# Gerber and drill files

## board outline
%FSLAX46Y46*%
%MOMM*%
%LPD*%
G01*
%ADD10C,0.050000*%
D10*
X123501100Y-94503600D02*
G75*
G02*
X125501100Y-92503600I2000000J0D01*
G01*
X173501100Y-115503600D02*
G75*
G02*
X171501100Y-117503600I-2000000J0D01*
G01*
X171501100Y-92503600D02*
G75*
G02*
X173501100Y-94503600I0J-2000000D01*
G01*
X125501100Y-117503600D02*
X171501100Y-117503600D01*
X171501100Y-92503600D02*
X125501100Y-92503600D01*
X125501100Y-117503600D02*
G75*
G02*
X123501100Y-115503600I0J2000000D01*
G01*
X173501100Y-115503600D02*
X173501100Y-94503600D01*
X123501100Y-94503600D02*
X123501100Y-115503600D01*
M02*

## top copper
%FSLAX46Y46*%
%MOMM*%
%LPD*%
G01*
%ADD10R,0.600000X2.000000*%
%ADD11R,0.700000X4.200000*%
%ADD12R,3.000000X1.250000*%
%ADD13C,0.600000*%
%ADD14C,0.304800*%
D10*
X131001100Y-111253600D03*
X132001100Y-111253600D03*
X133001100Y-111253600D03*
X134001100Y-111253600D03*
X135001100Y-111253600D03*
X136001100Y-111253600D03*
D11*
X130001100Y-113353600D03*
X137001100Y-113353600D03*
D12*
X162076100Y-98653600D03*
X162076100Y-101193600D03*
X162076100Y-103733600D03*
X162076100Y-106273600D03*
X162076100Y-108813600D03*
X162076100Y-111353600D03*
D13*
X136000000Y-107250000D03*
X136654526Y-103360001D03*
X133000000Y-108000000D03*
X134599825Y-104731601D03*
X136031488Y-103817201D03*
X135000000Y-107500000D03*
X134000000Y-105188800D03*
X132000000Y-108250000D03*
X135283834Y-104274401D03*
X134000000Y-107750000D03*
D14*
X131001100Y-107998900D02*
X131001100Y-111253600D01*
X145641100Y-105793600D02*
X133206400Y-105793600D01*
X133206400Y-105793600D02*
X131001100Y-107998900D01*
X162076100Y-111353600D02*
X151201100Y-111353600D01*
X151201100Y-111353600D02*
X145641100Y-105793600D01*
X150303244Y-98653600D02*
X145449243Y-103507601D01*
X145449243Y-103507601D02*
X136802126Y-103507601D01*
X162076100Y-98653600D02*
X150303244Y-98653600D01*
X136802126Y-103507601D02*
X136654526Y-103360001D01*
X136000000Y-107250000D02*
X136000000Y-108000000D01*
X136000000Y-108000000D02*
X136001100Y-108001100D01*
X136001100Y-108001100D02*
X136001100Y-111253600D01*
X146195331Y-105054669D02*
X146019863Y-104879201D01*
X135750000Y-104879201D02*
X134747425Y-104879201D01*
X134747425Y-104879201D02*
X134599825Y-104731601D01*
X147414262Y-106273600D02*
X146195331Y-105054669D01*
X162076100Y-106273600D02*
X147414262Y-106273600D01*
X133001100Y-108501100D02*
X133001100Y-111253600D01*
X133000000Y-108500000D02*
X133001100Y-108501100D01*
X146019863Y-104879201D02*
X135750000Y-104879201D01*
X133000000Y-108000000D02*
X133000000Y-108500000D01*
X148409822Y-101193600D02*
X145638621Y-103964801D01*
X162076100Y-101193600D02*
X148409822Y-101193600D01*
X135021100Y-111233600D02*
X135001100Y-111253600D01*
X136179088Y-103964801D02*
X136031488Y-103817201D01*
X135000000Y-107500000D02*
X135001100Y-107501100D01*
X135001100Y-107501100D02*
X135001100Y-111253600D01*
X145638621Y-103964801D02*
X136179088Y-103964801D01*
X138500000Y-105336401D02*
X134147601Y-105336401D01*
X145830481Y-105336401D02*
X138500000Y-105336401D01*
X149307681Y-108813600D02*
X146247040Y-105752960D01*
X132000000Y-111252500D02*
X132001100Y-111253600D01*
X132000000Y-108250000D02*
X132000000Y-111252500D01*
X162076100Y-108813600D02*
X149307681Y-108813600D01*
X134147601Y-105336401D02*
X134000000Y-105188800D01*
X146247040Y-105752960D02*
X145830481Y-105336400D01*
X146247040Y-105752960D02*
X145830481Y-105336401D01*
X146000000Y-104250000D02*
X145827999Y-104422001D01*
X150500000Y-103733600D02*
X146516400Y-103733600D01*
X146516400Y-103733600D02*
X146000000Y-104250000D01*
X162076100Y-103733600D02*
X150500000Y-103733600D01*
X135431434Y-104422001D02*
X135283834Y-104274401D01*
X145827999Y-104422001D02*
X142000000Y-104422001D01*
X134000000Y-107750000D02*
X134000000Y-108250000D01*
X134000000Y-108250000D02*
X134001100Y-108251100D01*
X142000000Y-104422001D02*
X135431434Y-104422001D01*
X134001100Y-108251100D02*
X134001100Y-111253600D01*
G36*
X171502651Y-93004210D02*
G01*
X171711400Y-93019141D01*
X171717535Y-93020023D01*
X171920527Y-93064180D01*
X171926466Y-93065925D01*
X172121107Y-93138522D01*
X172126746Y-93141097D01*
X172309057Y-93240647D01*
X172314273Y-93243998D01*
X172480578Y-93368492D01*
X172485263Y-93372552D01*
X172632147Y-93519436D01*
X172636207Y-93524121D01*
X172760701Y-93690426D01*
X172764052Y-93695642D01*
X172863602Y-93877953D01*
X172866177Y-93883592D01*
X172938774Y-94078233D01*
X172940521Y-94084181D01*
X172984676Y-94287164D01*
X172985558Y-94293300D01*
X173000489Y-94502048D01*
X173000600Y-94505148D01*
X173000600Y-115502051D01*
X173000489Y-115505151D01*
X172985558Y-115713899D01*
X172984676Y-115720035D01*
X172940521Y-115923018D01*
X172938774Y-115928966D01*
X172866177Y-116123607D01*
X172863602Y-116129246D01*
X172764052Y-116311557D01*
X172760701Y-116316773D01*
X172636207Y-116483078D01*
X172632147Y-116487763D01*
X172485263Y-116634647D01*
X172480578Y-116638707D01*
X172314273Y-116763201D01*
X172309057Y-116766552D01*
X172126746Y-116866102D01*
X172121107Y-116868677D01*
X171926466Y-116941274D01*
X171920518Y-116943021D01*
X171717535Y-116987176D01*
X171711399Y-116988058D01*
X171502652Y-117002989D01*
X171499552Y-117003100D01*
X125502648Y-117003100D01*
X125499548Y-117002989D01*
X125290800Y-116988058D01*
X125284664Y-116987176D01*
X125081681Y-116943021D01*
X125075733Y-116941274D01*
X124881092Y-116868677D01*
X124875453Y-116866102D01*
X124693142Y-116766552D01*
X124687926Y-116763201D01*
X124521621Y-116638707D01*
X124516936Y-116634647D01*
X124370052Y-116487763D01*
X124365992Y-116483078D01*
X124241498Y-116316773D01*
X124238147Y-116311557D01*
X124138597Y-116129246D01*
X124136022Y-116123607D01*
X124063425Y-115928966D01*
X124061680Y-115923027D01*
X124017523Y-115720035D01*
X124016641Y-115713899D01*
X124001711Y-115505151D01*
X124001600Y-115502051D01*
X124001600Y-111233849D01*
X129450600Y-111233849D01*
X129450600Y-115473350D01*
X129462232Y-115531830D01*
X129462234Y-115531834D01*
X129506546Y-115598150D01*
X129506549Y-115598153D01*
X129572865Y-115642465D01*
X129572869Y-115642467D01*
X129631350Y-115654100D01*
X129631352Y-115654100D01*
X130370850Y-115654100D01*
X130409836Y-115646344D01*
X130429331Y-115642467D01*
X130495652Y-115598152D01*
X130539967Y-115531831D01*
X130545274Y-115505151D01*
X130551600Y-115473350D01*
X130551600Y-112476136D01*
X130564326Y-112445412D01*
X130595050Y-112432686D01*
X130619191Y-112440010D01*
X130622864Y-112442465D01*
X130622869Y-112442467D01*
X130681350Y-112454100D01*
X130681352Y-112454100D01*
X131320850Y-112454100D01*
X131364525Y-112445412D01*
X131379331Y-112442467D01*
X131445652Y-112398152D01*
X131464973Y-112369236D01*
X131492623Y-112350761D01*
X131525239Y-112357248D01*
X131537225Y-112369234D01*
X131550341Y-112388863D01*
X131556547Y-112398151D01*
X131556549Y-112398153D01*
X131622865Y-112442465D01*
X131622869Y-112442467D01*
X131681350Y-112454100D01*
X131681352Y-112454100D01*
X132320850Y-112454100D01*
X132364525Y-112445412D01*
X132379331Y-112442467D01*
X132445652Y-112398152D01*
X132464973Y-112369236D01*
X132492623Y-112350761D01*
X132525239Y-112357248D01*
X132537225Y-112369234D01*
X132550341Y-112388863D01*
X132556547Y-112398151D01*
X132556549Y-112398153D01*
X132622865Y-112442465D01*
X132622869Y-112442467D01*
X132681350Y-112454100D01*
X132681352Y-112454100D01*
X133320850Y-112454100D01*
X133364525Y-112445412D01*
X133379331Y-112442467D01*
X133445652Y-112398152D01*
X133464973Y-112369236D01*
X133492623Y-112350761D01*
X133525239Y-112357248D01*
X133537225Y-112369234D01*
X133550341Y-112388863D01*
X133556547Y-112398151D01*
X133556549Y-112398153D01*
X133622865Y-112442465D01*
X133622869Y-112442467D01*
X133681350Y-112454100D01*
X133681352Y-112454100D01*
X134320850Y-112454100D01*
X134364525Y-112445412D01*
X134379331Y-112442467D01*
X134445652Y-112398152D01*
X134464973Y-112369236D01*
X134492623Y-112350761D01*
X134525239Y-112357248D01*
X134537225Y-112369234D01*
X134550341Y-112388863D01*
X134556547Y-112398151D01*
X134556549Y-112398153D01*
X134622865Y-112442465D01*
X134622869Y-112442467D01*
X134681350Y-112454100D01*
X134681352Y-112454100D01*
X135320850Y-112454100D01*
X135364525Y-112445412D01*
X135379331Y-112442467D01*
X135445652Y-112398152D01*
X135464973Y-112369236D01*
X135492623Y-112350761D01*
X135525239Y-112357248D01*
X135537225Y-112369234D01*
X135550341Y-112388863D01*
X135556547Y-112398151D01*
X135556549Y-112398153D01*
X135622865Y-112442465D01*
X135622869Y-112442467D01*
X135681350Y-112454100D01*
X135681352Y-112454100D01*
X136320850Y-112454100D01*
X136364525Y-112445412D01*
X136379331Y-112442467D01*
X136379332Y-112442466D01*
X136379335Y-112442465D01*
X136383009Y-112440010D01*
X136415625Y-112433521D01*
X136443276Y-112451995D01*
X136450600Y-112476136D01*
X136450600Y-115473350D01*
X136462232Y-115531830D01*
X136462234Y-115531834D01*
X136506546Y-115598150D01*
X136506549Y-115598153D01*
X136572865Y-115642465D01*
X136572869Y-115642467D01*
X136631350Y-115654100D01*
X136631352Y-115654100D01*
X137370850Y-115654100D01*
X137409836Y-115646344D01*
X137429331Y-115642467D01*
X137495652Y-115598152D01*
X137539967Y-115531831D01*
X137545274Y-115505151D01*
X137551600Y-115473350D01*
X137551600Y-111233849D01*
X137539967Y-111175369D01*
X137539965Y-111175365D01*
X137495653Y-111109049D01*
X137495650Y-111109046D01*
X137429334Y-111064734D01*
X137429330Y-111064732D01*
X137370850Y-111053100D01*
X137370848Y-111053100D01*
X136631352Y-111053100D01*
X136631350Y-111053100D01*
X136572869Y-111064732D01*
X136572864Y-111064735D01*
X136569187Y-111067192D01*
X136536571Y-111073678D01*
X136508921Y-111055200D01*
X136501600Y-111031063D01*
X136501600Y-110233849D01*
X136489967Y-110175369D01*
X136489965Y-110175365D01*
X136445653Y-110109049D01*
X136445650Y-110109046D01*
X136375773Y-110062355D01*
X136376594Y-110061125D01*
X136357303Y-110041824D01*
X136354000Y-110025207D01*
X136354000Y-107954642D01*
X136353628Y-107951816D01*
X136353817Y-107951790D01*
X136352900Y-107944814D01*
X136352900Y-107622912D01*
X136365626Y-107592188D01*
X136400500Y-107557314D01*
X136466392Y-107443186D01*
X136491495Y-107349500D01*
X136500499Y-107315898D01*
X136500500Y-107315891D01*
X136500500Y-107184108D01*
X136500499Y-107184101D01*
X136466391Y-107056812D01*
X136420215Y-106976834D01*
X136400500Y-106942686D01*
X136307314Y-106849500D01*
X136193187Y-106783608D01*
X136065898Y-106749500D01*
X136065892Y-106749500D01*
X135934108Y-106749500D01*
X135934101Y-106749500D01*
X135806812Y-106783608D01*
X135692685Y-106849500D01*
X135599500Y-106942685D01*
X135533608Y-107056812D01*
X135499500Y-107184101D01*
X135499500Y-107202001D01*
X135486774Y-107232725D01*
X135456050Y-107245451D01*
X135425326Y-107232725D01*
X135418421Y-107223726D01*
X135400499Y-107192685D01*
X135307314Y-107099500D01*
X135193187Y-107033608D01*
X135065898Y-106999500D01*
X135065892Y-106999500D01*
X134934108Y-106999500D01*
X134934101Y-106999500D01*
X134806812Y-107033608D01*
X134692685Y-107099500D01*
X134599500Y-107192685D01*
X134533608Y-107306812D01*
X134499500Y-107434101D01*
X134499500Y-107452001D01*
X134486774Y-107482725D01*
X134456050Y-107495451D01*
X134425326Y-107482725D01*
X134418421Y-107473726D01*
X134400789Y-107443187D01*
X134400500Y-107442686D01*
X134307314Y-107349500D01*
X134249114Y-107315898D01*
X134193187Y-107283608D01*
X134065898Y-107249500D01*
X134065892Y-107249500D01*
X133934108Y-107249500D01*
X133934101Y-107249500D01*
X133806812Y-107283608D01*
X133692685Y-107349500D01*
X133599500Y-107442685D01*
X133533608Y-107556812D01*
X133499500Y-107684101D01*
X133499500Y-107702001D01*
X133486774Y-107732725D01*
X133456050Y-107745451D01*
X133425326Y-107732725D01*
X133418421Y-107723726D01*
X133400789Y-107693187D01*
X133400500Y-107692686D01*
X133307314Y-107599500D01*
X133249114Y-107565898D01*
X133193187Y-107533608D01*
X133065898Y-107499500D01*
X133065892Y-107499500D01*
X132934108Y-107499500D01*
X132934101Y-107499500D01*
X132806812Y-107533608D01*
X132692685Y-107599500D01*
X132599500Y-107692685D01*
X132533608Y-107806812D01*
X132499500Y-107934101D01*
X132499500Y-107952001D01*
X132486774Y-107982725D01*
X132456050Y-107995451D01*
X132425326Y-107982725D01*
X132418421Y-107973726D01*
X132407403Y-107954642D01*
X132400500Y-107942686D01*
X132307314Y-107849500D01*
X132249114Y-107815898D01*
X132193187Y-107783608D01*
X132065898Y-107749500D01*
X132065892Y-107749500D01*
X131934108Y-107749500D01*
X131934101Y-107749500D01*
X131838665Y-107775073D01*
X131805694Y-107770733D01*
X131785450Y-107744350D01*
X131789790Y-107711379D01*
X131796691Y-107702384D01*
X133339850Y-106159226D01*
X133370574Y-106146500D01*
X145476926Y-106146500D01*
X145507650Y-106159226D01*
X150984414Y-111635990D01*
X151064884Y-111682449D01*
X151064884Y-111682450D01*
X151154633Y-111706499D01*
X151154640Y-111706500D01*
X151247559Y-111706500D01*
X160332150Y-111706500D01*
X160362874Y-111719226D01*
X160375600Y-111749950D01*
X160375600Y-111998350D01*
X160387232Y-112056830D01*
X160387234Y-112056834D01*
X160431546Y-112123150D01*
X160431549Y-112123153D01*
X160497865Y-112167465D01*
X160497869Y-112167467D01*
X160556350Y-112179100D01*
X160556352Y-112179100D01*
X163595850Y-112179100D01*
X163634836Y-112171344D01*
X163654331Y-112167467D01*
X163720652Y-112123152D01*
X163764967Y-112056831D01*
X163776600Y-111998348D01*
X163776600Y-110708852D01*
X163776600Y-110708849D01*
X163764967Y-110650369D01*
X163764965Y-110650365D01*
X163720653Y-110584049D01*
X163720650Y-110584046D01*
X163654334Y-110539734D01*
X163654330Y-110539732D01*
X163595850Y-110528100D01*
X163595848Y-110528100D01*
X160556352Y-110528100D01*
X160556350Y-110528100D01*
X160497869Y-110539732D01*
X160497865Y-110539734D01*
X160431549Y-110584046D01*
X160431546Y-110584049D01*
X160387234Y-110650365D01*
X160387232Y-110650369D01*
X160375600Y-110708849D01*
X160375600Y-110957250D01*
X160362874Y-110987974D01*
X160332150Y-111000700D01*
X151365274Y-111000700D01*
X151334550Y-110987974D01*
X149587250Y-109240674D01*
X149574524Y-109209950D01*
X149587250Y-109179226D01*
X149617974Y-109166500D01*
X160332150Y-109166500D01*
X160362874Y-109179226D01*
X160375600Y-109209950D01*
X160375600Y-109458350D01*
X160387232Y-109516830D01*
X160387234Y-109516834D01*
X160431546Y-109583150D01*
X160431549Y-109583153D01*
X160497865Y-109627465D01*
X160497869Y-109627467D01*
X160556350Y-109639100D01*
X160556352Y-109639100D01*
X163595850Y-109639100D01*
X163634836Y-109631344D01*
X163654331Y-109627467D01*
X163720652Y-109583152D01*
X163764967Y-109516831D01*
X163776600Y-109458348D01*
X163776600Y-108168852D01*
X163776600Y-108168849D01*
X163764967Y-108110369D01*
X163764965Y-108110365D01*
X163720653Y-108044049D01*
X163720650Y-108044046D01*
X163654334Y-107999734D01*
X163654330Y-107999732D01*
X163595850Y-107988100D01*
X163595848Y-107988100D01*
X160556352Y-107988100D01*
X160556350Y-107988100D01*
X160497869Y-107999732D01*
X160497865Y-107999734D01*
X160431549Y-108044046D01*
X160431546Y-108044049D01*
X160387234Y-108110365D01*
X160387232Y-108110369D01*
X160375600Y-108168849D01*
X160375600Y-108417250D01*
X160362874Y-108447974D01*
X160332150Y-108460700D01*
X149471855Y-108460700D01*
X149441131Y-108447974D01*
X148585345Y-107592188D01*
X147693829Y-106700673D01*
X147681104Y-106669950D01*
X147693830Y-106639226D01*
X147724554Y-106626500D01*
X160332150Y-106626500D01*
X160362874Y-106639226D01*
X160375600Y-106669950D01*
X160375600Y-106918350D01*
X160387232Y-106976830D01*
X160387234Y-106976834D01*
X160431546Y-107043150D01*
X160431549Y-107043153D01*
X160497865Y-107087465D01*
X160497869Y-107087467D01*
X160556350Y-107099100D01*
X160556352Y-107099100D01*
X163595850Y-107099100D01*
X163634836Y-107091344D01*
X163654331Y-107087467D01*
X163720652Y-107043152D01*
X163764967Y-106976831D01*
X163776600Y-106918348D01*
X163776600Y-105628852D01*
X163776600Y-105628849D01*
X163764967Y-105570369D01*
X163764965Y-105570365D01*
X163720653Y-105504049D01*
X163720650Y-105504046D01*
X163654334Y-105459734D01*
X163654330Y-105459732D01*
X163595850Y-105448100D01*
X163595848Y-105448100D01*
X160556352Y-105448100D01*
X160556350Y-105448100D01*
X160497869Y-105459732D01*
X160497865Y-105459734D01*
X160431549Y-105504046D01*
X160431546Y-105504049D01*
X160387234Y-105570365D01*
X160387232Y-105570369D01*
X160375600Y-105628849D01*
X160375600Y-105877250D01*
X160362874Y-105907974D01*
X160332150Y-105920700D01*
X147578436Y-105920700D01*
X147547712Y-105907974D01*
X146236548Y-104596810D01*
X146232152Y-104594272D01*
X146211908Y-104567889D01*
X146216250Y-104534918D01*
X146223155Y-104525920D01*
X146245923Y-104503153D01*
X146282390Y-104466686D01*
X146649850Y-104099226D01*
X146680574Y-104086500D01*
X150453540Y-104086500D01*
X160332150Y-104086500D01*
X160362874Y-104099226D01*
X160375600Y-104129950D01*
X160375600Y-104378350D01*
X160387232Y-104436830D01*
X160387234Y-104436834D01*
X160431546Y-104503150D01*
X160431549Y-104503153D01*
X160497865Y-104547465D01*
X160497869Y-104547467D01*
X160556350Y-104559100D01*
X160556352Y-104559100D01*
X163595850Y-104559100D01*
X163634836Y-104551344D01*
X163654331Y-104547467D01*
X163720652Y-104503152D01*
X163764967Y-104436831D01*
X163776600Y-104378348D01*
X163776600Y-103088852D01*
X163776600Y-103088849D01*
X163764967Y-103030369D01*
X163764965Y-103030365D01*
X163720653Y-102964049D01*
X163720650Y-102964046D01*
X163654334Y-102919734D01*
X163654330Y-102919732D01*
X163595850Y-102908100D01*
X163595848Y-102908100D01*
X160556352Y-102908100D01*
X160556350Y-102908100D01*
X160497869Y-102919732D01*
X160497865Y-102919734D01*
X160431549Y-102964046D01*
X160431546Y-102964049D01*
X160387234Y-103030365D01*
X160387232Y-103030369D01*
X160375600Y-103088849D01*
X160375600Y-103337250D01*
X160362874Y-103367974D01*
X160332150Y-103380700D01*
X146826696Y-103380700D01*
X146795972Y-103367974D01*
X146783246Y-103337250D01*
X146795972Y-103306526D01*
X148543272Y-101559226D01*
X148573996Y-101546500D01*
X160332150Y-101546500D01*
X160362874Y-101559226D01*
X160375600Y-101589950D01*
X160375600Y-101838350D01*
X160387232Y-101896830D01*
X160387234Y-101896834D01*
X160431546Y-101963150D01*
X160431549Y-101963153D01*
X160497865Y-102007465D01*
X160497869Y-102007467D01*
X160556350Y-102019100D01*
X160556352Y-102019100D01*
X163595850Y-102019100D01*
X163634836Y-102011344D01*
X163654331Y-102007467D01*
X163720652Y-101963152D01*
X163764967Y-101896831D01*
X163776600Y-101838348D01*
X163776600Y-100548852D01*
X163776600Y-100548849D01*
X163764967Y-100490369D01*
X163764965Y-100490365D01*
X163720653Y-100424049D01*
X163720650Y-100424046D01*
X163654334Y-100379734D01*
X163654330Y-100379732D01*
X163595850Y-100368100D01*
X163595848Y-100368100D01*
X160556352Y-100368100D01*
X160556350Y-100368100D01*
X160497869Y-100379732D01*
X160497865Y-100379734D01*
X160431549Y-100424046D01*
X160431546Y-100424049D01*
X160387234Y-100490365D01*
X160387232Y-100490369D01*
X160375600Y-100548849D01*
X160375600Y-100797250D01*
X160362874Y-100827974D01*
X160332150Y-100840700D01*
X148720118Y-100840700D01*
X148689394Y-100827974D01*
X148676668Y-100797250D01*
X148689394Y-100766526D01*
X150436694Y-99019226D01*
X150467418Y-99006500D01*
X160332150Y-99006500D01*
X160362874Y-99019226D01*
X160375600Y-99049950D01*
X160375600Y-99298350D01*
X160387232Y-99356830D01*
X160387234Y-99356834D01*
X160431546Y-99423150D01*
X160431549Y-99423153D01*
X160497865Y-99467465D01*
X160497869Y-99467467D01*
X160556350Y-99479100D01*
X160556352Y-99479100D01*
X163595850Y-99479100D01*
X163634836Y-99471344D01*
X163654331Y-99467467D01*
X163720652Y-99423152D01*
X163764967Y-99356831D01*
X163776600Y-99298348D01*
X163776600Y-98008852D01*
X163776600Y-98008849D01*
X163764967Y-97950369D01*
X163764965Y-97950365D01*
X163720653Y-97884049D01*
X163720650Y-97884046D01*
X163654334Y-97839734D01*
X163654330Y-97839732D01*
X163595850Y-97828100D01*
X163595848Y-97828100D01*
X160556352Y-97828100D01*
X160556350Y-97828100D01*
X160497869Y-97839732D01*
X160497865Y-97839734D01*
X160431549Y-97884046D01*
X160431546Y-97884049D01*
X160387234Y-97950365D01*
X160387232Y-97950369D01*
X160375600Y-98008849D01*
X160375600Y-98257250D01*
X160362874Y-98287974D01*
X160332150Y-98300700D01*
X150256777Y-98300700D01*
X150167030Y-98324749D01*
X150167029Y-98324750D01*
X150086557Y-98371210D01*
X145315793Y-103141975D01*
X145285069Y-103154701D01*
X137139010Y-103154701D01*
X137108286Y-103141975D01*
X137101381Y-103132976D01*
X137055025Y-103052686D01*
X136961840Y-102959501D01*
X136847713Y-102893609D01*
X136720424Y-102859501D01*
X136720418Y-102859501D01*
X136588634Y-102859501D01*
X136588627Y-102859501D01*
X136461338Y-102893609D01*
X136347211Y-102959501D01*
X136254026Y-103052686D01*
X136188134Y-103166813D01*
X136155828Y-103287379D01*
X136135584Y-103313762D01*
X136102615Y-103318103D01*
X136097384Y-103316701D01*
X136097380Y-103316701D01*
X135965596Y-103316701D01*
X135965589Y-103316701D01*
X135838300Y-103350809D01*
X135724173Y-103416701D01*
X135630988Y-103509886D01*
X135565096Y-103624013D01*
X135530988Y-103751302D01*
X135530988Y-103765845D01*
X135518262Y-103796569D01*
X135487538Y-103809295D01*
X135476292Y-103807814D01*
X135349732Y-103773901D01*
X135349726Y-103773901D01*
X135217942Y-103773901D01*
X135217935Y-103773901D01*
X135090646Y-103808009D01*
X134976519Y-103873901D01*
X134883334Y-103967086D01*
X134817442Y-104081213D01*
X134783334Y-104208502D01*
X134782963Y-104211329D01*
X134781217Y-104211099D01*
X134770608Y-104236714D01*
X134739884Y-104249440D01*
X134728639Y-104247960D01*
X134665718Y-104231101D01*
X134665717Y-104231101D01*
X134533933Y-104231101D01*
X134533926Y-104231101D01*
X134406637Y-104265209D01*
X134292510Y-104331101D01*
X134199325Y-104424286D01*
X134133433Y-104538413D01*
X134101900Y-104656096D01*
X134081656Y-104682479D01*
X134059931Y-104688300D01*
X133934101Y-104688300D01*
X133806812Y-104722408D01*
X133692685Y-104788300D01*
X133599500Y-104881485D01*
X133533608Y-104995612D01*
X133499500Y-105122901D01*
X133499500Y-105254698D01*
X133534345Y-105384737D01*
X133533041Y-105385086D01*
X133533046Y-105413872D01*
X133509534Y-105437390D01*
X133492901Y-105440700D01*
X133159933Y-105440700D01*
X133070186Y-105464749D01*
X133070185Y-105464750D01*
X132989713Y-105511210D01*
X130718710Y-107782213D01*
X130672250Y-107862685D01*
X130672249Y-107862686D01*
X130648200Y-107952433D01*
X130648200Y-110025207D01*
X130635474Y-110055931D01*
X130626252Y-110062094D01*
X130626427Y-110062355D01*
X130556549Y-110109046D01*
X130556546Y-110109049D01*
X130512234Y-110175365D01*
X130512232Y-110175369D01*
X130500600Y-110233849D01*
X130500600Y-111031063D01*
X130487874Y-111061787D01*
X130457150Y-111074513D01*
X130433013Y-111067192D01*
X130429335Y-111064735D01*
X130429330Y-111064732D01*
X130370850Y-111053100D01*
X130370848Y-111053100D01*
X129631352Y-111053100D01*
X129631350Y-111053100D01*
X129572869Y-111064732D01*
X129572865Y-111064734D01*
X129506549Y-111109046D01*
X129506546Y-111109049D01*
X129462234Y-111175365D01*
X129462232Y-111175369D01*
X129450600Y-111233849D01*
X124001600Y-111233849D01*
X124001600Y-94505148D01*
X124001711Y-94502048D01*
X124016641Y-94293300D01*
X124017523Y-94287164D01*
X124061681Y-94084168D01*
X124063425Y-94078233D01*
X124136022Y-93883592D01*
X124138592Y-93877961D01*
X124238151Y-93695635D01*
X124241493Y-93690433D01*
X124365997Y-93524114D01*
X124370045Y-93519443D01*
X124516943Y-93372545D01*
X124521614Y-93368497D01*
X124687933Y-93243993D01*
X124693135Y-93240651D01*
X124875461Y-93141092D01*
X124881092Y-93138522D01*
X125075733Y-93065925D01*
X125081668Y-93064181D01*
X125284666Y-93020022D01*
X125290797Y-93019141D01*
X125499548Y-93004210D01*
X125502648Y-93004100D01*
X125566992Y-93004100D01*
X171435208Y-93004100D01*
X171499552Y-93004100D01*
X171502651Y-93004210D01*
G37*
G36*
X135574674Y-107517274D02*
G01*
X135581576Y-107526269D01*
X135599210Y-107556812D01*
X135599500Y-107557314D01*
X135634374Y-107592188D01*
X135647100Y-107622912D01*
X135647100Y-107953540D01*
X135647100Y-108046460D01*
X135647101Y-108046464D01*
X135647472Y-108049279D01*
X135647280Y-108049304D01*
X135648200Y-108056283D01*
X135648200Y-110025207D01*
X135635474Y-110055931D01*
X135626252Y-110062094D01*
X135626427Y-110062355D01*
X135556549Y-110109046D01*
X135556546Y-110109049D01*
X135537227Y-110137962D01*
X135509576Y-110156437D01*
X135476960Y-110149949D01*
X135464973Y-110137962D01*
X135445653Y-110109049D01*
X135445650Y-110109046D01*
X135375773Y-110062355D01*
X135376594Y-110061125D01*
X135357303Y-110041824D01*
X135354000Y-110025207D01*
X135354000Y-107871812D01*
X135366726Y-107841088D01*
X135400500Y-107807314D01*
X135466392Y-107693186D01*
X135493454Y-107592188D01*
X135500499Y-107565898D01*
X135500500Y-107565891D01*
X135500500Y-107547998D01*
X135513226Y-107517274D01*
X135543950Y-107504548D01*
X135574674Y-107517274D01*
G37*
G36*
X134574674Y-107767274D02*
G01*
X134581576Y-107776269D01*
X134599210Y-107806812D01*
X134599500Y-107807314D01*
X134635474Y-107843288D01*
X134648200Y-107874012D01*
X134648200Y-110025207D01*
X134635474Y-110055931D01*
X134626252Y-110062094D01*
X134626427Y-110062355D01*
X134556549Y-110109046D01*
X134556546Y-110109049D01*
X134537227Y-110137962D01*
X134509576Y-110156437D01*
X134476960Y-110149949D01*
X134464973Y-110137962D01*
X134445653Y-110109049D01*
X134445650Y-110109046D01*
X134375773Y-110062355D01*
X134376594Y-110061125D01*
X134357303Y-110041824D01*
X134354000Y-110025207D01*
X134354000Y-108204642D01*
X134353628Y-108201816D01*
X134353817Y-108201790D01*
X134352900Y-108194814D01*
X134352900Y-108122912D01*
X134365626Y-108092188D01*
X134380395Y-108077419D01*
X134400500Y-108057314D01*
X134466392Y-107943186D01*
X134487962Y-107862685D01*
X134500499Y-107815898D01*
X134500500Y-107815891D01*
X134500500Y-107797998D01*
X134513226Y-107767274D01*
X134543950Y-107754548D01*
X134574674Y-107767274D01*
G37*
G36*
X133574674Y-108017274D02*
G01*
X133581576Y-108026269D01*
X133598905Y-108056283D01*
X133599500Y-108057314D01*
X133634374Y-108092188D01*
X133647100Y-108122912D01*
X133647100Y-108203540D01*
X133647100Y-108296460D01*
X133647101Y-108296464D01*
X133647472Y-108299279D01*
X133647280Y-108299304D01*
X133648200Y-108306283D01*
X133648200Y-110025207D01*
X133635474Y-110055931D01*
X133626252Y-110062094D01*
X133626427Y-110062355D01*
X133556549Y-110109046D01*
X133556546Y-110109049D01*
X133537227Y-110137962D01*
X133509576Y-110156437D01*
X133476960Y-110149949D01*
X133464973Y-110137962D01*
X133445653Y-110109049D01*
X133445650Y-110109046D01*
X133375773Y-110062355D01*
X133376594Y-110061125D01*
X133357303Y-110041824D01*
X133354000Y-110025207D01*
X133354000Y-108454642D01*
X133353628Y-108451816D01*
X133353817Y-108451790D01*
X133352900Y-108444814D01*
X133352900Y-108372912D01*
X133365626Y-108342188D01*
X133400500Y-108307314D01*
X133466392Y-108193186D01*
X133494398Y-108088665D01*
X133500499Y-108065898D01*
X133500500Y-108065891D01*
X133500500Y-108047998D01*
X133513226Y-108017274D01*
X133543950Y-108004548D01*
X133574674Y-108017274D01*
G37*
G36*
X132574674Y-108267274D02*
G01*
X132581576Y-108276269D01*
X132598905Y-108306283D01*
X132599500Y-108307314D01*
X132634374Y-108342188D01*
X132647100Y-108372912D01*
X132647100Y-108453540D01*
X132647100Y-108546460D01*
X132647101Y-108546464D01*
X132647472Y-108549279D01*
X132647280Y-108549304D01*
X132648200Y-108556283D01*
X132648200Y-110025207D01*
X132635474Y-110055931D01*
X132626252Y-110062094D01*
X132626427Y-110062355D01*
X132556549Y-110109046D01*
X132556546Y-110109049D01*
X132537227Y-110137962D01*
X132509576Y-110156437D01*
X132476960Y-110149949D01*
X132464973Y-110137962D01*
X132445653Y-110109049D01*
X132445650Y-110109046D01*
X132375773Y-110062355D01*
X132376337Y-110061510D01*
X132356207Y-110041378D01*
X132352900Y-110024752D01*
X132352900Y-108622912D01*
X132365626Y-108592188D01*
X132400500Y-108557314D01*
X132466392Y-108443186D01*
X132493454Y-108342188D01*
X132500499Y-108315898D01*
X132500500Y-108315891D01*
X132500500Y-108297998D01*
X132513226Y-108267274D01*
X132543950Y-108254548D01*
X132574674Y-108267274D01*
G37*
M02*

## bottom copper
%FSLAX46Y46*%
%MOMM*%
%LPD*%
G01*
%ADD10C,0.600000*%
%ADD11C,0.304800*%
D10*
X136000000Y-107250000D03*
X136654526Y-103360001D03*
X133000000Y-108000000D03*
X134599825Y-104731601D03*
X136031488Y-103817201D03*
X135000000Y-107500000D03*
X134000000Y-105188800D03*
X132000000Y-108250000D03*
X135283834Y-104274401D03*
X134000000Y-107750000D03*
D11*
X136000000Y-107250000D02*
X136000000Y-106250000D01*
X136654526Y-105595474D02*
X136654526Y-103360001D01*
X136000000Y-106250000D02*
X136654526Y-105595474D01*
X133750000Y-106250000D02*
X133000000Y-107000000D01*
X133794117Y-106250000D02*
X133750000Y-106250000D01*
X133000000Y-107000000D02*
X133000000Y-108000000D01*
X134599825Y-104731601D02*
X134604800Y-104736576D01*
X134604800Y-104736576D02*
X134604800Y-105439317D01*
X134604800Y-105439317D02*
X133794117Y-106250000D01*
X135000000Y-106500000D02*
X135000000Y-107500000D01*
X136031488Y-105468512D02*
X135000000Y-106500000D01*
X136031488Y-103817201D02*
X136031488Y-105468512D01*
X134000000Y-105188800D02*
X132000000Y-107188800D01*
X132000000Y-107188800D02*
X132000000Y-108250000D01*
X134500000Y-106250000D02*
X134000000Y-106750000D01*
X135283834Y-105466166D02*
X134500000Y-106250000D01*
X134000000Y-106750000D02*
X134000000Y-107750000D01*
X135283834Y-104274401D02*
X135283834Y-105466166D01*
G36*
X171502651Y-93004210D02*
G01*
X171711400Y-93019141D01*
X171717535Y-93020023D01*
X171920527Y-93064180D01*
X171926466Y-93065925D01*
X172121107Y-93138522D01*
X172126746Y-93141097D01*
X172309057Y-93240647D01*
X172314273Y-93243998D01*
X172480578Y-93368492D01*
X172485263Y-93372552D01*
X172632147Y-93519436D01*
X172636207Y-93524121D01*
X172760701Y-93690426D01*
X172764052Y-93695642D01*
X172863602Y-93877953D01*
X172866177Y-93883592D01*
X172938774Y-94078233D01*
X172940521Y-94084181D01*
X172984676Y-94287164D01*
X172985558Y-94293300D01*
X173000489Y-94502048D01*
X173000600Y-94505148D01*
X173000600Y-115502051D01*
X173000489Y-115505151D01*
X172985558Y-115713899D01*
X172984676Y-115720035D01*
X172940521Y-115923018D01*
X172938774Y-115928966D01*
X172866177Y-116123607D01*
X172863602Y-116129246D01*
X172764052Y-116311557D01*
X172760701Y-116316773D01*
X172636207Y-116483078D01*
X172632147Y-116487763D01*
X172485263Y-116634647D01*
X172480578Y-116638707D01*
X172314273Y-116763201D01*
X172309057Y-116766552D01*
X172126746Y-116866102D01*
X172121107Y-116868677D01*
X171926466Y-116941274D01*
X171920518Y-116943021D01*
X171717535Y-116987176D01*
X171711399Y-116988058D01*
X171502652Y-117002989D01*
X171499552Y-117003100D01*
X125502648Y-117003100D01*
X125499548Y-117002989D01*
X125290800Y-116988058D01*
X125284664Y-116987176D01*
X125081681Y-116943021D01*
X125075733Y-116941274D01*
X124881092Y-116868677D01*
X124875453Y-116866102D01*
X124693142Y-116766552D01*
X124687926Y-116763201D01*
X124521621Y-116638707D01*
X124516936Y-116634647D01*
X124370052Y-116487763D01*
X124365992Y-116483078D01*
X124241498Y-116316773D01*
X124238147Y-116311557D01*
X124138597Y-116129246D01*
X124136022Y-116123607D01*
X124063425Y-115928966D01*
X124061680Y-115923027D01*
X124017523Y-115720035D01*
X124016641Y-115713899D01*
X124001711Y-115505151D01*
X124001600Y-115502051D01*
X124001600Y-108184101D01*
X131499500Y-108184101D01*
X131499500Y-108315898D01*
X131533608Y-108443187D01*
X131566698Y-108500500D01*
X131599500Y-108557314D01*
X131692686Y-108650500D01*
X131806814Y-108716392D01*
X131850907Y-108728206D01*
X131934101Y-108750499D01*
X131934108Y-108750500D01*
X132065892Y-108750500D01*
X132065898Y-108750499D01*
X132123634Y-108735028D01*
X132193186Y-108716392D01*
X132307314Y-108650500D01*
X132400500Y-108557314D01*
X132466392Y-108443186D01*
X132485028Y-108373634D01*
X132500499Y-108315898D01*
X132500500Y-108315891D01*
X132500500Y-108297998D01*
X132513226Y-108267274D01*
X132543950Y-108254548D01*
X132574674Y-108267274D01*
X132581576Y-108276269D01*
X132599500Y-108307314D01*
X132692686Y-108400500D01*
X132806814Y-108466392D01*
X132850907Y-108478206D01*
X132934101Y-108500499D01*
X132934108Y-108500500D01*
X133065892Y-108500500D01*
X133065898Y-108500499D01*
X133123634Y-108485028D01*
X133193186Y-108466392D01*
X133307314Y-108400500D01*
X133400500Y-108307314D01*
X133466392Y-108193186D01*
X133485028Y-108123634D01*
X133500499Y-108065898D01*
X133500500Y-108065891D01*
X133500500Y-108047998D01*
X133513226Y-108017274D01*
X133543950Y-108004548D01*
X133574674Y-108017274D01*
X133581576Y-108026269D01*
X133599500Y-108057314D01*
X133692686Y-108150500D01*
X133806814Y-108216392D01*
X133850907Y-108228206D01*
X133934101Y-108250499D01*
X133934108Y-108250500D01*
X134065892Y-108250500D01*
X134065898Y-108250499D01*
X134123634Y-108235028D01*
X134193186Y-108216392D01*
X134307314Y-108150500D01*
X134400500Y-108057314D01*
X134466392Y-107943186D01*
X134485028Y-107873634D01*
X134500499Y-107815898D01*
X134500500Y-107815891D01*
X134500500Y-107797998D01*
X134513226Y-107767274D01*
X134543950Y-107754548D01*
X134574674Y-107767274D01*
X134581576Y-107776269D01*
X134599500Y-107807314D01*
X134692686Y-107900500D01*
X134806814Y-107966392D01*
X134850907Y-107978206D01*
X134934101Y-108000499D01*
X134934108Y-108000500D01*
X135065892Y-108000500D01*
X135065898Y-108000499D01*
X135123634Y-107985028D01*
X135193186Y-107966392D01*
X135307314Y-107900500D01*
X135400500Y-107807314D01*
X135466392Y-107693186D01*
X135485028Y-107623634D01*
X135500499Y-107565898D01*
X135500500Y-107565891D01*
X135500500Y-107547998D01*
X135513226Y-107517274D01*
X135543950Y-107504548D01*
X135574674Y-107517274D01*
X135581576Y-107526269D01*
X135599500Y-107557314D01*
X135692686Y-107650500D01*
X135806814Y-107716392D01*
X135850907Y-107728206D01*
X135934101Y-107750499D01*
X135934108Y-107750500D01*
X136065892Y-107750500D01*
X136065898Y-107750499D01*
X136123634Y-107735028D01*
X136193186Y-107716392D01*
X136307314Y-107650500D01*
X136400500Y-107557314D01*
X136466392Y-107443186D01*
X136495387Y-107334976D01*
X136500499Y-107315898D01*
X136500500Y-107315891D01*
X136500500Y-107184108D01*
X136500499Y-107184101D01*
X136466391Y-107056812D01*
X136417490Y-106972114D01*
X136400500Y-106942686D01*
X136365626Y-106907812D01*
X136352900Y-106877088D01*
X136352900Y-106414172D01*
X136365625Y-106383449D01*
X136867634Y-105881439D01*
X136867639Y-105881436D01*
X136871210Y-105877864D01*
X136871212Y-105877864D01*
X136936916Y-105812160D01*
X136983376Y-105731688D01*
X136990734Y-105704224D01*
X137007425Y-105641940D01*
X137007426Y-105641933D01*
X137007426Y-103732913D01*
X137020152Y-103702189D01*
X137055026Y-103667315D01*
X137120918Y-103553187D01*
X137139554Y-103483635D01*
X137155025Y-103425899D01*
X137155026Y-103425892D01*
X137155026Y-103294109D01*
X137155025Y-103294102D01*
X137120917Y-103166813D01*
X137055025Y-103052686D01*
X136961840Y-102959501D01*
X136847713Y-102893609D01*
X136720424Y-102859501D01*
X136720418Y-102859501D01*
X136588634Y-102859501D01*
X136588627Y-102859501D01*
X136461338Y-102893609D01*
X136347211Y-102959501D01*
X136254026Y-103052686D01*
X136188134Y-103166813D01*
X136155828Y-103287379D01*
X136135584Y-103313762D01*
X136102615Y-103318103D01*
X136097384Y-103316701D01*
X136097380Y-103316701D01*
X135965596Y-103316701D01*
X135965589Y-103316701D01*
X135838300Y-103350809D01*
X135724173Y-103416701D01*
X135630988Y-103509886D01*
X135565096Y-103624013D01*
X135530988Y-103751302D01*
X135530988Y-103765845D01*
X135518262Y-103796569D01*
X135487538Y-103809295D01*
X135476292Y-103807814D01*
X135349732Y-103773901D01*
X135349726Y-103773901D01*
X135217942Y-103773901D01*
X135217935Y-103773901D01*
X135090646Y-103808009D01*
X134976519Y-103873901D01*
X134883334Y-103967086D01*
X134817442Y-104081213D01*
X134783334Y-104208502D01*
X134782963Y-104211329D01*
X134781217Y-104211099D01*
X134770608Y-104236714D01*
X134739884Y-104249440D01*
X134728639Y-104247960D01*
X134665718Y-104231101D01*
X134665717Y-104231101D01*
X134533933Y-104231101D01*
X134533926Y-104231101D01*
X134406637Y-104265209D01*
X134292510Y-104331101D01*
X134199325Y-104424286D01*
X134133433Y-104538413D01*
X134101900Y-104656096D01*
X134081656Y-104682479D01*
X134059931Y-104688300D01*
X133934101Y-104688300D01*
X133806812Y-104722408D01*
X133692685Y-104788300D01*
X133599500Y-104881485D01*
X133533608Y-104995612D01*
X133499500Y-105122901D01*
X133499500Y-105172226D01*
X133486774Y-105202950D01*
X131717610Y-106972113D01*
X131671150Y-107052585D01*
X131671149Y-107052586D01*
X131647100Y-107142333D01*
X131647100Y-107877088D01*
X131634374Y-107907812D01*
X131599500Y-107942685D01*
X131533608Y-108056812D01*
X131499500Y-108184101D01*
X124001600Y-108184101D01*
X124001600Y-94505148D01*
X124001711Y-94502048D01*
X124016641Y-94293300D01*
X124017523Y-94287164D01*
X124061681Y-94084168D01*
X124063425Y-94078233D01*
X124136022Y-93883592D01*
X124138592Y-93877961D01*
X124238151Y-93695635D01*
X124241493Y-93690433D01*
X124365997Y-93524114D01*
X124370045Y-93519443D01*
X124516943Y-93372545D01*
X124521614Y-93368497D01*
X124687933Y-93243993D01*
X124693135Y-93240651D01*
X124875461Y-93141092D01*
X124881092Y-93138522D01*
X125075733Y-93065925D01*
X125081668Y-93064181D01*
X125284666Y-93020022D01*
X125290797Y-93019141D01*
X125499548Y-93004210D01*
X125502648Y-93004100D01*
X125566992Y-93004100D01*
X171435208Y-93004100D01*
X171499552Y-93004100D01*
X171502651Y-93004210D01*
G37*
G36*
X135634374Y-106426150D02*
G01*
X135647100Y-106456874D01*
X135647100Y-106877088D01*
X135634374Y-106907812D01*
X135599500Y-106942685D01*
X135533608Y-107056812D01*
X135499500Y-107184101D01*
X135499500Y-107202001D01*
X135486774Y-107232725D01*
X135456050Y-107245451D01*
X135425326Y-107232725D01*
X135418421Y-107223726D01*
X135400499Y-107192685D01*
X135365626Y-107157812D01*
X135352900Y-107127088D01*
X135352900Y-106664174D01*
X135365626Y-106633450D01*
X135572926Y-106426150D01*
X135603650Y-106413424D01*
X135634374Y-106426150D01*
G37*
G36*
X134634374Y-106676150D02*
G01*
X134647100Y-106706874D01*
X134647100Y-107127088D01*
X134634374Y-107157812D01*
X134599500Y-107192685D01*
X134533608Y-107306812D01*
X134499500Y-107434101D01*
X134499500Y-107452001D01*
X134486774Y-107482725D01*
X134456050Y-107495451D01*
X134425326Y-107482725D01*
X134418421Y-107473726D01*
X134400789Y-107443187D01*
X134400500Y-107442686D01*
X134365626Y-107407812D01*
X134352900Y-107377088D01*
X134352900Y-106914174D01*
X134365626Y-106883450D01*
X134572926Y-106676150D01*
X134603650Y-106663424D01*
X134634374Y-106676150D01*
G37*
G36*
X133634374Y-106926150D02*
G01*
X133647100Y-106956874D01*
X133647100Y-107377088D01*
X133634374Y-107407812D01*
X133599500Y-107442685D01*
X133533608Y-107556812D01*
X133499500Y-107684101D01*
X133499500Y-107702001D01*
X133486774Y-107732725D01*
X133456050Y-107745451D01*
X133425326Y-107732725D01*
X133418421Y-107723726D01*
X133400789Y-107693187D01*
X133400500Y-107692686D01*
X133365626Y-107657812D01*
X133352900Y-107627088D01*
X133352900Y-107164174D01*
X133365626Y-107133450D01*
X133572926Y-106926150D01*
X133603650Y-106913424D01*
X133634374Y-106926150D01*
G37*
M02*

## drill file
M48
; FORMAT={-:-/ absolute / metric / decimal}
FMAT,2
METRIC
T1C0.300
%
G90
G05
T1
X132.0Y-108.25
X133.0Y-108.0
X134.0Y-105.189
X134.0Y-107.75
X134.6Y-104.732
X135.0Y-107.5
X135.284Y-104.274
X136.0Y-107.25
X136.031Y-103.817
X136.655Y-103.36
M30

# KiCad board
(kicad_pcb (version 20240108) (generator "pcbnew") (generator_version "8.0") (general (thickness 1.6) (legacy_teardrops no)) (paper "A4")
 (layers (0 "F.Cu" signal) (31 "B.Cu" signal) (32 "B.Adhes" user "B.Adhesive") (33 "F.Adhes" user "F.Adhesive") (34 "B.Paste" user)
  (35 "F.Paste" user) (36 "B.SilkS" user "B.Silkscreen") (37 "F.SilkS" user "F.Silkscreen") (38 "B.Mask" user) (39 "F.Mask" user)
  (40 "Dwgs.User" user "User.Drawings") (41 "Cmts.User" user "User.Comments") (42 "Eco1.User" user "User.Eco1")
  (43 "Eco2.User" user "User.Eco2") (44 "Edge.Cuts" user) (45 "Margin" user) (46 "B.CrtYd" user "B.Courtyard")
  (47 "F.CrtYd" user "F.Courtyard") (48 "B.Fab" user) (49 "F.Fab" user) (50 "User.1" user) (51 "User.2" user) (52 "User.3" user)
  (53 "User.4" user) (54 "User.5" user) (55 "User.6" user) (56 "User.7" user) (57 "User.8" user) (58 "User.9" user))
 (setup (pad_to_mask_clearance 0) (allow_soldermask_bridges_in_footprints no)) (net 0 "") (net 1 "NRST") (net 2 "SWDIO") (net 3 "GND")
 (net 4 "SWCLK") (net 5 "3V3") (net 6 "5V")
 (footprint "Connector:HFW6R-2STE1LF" (layer "F.Cu") (at 133.5011 114.5036)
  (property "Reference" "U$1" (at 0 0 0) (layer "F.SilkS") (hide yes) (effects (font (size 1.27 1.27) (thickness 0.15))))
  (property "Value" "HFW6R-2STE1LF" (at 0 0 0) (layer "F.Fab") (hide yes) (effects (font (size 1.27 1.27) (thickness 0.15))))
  (pad "P$1" smd rect (at -2.5 -3.25) (size 0.6 2) (layers "F.Cu" "F.Paste" "F.Mask") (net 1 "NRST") (solder_mask_margin 0.0508)
   (thermal_bridge_angle 0))
  (pad "P$2" smd rect (at -1.5 -3.25) (size 0.6 2) (layers "F.Cu" "F.Paste" "F.Mask") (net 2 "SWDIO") (solder_mask_margin 0.0508)
   (thermal_bridge_angle 0))
  (pad "P$3" smd rect (at -0.5 -3.25) (size 0.6 2) (layers "F.Cu" "F.Paste" "F.Mask") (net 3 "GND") (solder_mask_margin 0.0508)
   (thermal_bridge_angle 0))
  (pad "P$4" smd rect (at 0.5 -3.25) (size 0.6 2) (layers "F.Cu" "F.Paste" "F.Mask") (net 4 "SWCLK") (solder_mask_margin 0.0508)
   (thermal_bridge_angle 0))
  (pad "P$5" smd rect (at 1.5 -3.25) (size 0.6 2) (layers "F.Cu" "F.Paste" "F.Mask") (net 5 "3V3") (solder_mask_margin 0.0508)
   (thermal_bridge_angle 0))
  (pad "P$6" smd rect (at 2.5 -3.25) (size 0.6 2) (layers "F.Cu" "F.Paste" "F.Mask") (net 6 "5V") (solder_mask_margin 0.0508)
   (thermal_bridge_angle 0))
  (pad "P$7" smd rect (at -3.5 -1.15) (size 0.7 4.2) (layers "F.Cu" "F.Paste" "F.Mask") (solder_mask_margin 0.0508) (thermal_bridge_angle 0))
  (pad "P$8" smd rect (at 3.5 -1.15) (size 0.7 4.2) (layers "F.Cu" "F.Paste" "F.Mask") (solder_mask_margin 0.0508) (thermal_bridge_angle 0)))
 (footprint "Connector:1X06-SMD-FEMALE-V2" (layer "F.Cu") (at 165.5011 105.0036 90)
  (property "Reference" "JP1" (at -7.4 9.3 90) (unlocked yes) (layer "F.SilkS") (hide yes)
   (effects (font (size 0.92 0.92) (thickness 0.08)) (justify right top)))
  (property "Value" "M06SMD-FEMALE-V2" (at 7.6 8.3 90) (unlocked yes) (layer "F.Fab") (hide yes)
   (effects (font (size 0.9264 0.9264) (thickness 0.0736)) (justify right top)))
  (pad "1" smd rect (at 6.35 -3.425 270) (size 1.25 3) (layers "F.Cu" "F.Paste" "F.Mask") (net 6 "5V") (solder_mask_margin 0.0508)
   (thermal_bridge_angle 0))
  (pad "2" smd rect (at 3.81 -3.425 270) (size 1.25 3) (layers "F.Cu" "F.Paste" "F.Mask") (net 5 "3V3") (solder_mask_margin 0.0508)
   (thermal_bridge_angle 0))
  (pad "3" smd rect (at 1.27 -3.425 270) (size 1.25 3) (layers "F.Cu" "F.Paste" "F.Mask") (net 4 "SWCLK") (solder_mask_margin 0.0508)
   (thermal_bridge_angle 0))
  (pad "4" smd rect (at -1.27 -3.425 270) (size 1.25 3) (layers "F.Cu" "F.Paste" "F.Mask") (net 3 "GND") (solder_mask_margin 0.0508)
   (thermal_bridge_angle 0))
  (pad "5" smd rect (at -3.81 -3.425 270) (size 1.25 3) (layers "F.Cu" "F.Paste" "F.Mask") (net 2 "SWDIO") (solder_mask_margin 0.0508)
   (thermal_bridge_angle 0))
  (pad "6" smd rect (at -6.35 -3.425 270) (size 1.25 3) (layers "F.Cu" "F.Paste" "F.Mask") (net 1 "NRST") (solder_mask_margin 0.0508)
   (thermal_bridge_angle 0)))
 (gr_arc (start 123.5011 94.5036) (mid 124.086886 93.089386) (end 125.5011 92.5036) (stroke (width 0.05) (type solid)) (layer "Edge.Cuts"))
 (gr_arc (start 173.5011 115.5036) (mid 172.915314 116.917814) (end 171.5011 117.5036) (stroke (width 0.05) (type solid))
  (layer "Edge.Cuts"))
 (gr_arc (start 171.5011 92.5036) (mid 172.915314 93.089386) (end 173.5011 94.5036) (stroke (width 0.05) (type solid)) (layer "Edge.Cuts"))
 (gr_line (start 125.5011 117.5036) (end 171.5011 117.5036) (stroke (width 0.05) (type solid)) (layer "Edge.Cuts"))
 (gr_line (start 171.5011 92.5036) (end 125.5011 92.5036) (stroke (width 0.05) (type solid)) (layer "Edge.Cuts"))
 (gr_arc (start 125.5011 117.5036) (mid 124.086886 116.917814) (end 123.5011 115.5036) (stroke (width 0.05) (type solid))
  (layer "Edge.Cuts"))
 (gr_line (start 173.5011 115.5036) (end 173.5011 94.5036) (stroke (width 0.05) (type solid)) (layer "Edge.Cuts"))
 (gr_line (start 123.5011 94.5036) (end 123.5011 115.5036) (stroke (width 0.05) (type solid)) (layer "Edge.Cuts"))
 (segment (start 131.0011 107.9989) (end 131.0011 111.2536) (width 0.3048) (layer "F.Cu") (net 1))
 (segment (start 145.6411 105.7936) (end 133.2064 105.7936) (width 0.3048) (layer "F.Cu") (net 1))
 (segment (start 133.2064 105.7936) (end 131.0011 107.9989) (width 0.3048) (layer "F.Cu") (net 1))
 (segment (start 162.0761 111.3536) (end 151.2011 111.3536) (width 0.3048) (layer "F.Cu") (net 1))
 (segment (start 151.2011 111.3536) (end 145.6411 105.7936) (width 0.3048) (layer "F.Cu") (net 1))
 (segment (start 150.303244 98.6536) (end 145.449243 103.507601) (width 0.3048) (layer "F.Cu") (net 6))
 (segment (start 145.449243 103.507601) (end 136.802126 103.507601) (width 0.3048) (layer "F.Cu") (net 6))
 (segment (start 162.0761 98.6536) (end 150.303244 98.6536) (width 0.3048) (layer "F.Cu") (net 6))
 (segment (start 136.802126 103.507601) (end 136.654526 103.360001) (width 0.3048) (layer "F.Cu") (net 6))
 (segment (start 136 107.25) (end 136 108) (width 0.3048) (layer "F.Cu") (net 6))
 (segment (start 136 108) (end 136.0011 108.0011) (width 0.3048) (layer "F.Cu") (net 6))
 (segment (start 136.0011 108.0011) (end 136.0011 111.2536) (width 0.3048) (layer "F.Cu") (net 6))
 (via (at 136 107.25) (size 0.6) (drill 0.3) (layers "F.Cu" "B.Cu") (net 6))
 (via (at 136.654526 103.360001) (size 0.6) (drill 0.3) (layers "F.Cu" "B.Cu") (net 6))
 (segment (start 136 107.25) (end 136 106.25) (width 0.3048) (layer "B.Cu") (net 6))
 (segment (start 136.654526 105.595474) (end 136.654526 103.360001) (width 0.3048) (layer "B.Cu") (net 6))
 (segment (start 136 106.25) (end 136.654526 105.595474) (width 0.3048) (layer "B.Cu") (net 6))
 (segment (start 146.195331 105.054669) (end 146.019863 104.879201) (width 0.3048) (layer "F.Cu") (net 3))
 (segment (start 135.75 104.879201) (end 134.747425 104.879201) (width 0.3048) (layer "F.Cu") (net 3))
 (segment (start 134.747425 104.879201) (end 134.599825 104.731601) (width 0.3048) (layer "F.Cu") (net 3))
 (segment (start 147.414262 106.2736) (end 146.195331 105.054669) (width 0.3048) (layer "F.Cu") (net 3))
 (segment (start 162.0761 106.2736) (end 147.414262 106.2736) (width 0.3048) (layer "F.Cu") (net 3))
 (segment (start 133.0011 108.5011) (end 133.0011 111.2536) (width 0.3048) (layer "F.Cu") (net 3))
 (segment (start 133 108.5) (end 133.0011 108.5011) (width 0.3048) (layer "F.Cu") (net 3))
 (segment (start 146.019863 104.879201) (end 135.75 104.879201) (width 0.3048) (layer "F.Cu") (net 3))
 (segment (start 133 108) (end 133 108.5) (width 0.3048) (layer "F.Cu") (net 3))
 (via (at 133 108) (size 0.6) (drill 0.3) (layers "F.Cu" "B.Cu") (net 3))
 (via (at 134.599825 104.731601) (size 0.6) (drill 0.3) (layers "F.Cu" "B.Cu") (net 3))
 (segment (start 133.75 106.25) (end 133 107) (width 0.3048) (layer "B.Cu") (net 3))
 (segment (start 133.794117 106.25) (end 133.75 106.25) (width 0.3048) (layer "B.Cu") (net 3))
 (segment (start 133 107) (end 133 108) (width 0.3048) (layer "B.Cu") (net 3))
 (segment (start 134.599825 104.731601) (end 134.6048 104.736576) (width 0.3048) (layer "B.Cu") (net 3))
 (segment (start 134.6048 104.736576) (end 134.6048 105.439317) (width 0.3048) (layer "B.Cu") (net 3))
 (segment (start 134.6048 105.439317) (end 133.794117 106.25) (width 0.3048) (layer "B.Cu") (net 3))
 (segment (start 148.409822 101.1936) (end 145.638621 103.964801) (width 0.3048) (layer "F.Cu") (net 5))
 (segment (start 162.0761 101.1936) (end 148.409822 101.1936) (width 0.3048) (layer "F.Cu") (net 5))
 (segment (start 135.0211 111.2336) (end 135.0011 111.2536) (width 0.3048) (layer "F.Cu") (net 5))
 (segment (start 136.179088 103.964801) (end 136.031488 103.817201) (width 0.3048) (layer "F.Cu") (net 5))
 (segment (start 135 107.5) (end 135.0011 107.5011) (width 0.3048) (layer "F.Cu") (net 5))
 (segment (start 135.0011 107.5011) (end 135.0011 111.2536) (width 0.3048) (layer "F.Cu") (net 5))
 (segment (start 145.638621 103.964801) (end 136.179088 103.964801) (width 0.3048) (layer "F.Cu") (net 5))
 (via (at 136.031488 103.817201) (size 0.6) (drill 0.3) (layers "F.Cu" "B.Cu") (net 5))
 (via (at 135 107.5) (size 0.6) (drill 0.3) (layers "F.Cu" "B.Cu") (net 5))
 (segment (start 135 106.5) (end 135 107.5) (width 0.3048) (layer "B.Cu") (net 5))
 (segment (start 136.031488 105.468512) (end 135 106.5) (width 0.3048) (layer "B.Cu") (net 5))
 (segment (start 136.031488 103.817201) (end 136.031488 105.468512) (width 0.3048) (layer "B.Cu") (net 5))
 (segment (start 138.5 105.336401) (end 134.147601 105.336401) (width 0.3048) (layer "F.Cu") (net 2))
 (segment (start 145.830481 105.336401) (end 138.5 105.336401) (width 0.3048) (layer "F.Cu") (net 2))
 (segment (start 149.307681 108.8136) (end 146.24704 105.75296) (width 0.3048) (layer "F.Cu") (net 2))
 (segment (start 132 111.2525) (end 132.0011 111.2536) (width 0.3048) (layer "F.Cu") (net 2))
 (segment (start 132 108.25) (end 132 111.2525) (width 0.3048) (layer "F.Cu") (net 2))
 (segment (start 162.0761 108.8136) (end 149.307681 108.8136) (width 0.3048) (layer "F.Cu") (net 2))
 (segment (start 134.147601 105.336401) (end 134 105.1888) (width 0.3048) (layer "F.Cu") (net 2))
 (segment (start 146.24704 105.75296) (end 145.830481 105.3364) (width 0.3048) (layer "F.Cu") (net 2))
 (segment (start 146.24704 105.75296) (end 145.830481 105.336401) (width 0.3048) (layer "F.Cu") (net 2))
 (via (at 134 105.1888) (size 0.6) (drill 0.3) (layers "F.Cu" "B.Cu") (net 2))
 (via (at 132 108.25) (size 0.6) (drill 0.3) (layers "F.Cu" "B.Cu") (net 2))
 (segment (start 134 105.1888) (end 132 107.1888) (width 0.3048) (layer "B.Cu") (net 2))
 (segment (start 132 107.1888) (end 132 108.25) (width 0.3048) (layer "B.Cu") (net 2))
 (segment (start 146 104.25) (end 145.827999 104.422001) (width 0.3048) (layer "F.Cu") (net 4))
 (segment (start 150.5 103.7336) (end 146.5164 103.7336) (width 0.3048) (layer "F.Cu") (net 4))
 (segment (start 146.5164 103.7336) (end 146 104.25) (width 0.3048) (layer "F.Cu") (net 4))
 (segment (start 162.0761 103.7336) (end 150.5 103.7336) (width 0.3048) (layer "F.Cu") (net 4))
 (segment (start 135.431434 104.422001) (end 135.283834 104.274401) (width 0.3048) (layer "F.Cu") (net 4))
 (segment (start 145.827999 104.422001) (end 142 104.422001) (width 0.3048) (layer "F.Cu") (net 4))
 (segment (start 134 107.75) (end 134 108.25) (width 0.3048) (layer "F.Cu") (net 4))
 (segment (start 134 108.25) (end 134.0011 108.2511) (width 0.3048) (layer "F.Cu") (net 4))
 (segment (start 142 104.422001) (end 135.431434 104.422001) (width 0.3048) (layer "F.Cu") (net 4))
 (segment (start 134.0011 108.2511) (end 134.0011 111.2536) (width 0.3048) (layer "F.Cu") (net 4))
 (via (at 135.283834 104.274401) (size 0.6) (drill 0.3) (layers "F.Cu" "B.Cu") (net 4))
 (via (at 134 107.75) (size 0.6) (drill 0.3) (layers "F.Cu" "B.Cu") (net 4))
 (segment (start 134.5 106.25) (end 134 106.75) (width 0.3048) (layer "B.Cu") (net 4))
 (segment (start 135.283834 105.466166) (end 134.5 106.25) (width 0.3048) (layer "B.Cu") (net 4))
 (segment (start 134 106.75) (end 134 107.75) (width 0.3048) (layer "B.Cu") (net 4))
 (segment (start 135.283834 104.274401) (end 135.283834 105.466166) (width 0.3048) (layer "B.Cu") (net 4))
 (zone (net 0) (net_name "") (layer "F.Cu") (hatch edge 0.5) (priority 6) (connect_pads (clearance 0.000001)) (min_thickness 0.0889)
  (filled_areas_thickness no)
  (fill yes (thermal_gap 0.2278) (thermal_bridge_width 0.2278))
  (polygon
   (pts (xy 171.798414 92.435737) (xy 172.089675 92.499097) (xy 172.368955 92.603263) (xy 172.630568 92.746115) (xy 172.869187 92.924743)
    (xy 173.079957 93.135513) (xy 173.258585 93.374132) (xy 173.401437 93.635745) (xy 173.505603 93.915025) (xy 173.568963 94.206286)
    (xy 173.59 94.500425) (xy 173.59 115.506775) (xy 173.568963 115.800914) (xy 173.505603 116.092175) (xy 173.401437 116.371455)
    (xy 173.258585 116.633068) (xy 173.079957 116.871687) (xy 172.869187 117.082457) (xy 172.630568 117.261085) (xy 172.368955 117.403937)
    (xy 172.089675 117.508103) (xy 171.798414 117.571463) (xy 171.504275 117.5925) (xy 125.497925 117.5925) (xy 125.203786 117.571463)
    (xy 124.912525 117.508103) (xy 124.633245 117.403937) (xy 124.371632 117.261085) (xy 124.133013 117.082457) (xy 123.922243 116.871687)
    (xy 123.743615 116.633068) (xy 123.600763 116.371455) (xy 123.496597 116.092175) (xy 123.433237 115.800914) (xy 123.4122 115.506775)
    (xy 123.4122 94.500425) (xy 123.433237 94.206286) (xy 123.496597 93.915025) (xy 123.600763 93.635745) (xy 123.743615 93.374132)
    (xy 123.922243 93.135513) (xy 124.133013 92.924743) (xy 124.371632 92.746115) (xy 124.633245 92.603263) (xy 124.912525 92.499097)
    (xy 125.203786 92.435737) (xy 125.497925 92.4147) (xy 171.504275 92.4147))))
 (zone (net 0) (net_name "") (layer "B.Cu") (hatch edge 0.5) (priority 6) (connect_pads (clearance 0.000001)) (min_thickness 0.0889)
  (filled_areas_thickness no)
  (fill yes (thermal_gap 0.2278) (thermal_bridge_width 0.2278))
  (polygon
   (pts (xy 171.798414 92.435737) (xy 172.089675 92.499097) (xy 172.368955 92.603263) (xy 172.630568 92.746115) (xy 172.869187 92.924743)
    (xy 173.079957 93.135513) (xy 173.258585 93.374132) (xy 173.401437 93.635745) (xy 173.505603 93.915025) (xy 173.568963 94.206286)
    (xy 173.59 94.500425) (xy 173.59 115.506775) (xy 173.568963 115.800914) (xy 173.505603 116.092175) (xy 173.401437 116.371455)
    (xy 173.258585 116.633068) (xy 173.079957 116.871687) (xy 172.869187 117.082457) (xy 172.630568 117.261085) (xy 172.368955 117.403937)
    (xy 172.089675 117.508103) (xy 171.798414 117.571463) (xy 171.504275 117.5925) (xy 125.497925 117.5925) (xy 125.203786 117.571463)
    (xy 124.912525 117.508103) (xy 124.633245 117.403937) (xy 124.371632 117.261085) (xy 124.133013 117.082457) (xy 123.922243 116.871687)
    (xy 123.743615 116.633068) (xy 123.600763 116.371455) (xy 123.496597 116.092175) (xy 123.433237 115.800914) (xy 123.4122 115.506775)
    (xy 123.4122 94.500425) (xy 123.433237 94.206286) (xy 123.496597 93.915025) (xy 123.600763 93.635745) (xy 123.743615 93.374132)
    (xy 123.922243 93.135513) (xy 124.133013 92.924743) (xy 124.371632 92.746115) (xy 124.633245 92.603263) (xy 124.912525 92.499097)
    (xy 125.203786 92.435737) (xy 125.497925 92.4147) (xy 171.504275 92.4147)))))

